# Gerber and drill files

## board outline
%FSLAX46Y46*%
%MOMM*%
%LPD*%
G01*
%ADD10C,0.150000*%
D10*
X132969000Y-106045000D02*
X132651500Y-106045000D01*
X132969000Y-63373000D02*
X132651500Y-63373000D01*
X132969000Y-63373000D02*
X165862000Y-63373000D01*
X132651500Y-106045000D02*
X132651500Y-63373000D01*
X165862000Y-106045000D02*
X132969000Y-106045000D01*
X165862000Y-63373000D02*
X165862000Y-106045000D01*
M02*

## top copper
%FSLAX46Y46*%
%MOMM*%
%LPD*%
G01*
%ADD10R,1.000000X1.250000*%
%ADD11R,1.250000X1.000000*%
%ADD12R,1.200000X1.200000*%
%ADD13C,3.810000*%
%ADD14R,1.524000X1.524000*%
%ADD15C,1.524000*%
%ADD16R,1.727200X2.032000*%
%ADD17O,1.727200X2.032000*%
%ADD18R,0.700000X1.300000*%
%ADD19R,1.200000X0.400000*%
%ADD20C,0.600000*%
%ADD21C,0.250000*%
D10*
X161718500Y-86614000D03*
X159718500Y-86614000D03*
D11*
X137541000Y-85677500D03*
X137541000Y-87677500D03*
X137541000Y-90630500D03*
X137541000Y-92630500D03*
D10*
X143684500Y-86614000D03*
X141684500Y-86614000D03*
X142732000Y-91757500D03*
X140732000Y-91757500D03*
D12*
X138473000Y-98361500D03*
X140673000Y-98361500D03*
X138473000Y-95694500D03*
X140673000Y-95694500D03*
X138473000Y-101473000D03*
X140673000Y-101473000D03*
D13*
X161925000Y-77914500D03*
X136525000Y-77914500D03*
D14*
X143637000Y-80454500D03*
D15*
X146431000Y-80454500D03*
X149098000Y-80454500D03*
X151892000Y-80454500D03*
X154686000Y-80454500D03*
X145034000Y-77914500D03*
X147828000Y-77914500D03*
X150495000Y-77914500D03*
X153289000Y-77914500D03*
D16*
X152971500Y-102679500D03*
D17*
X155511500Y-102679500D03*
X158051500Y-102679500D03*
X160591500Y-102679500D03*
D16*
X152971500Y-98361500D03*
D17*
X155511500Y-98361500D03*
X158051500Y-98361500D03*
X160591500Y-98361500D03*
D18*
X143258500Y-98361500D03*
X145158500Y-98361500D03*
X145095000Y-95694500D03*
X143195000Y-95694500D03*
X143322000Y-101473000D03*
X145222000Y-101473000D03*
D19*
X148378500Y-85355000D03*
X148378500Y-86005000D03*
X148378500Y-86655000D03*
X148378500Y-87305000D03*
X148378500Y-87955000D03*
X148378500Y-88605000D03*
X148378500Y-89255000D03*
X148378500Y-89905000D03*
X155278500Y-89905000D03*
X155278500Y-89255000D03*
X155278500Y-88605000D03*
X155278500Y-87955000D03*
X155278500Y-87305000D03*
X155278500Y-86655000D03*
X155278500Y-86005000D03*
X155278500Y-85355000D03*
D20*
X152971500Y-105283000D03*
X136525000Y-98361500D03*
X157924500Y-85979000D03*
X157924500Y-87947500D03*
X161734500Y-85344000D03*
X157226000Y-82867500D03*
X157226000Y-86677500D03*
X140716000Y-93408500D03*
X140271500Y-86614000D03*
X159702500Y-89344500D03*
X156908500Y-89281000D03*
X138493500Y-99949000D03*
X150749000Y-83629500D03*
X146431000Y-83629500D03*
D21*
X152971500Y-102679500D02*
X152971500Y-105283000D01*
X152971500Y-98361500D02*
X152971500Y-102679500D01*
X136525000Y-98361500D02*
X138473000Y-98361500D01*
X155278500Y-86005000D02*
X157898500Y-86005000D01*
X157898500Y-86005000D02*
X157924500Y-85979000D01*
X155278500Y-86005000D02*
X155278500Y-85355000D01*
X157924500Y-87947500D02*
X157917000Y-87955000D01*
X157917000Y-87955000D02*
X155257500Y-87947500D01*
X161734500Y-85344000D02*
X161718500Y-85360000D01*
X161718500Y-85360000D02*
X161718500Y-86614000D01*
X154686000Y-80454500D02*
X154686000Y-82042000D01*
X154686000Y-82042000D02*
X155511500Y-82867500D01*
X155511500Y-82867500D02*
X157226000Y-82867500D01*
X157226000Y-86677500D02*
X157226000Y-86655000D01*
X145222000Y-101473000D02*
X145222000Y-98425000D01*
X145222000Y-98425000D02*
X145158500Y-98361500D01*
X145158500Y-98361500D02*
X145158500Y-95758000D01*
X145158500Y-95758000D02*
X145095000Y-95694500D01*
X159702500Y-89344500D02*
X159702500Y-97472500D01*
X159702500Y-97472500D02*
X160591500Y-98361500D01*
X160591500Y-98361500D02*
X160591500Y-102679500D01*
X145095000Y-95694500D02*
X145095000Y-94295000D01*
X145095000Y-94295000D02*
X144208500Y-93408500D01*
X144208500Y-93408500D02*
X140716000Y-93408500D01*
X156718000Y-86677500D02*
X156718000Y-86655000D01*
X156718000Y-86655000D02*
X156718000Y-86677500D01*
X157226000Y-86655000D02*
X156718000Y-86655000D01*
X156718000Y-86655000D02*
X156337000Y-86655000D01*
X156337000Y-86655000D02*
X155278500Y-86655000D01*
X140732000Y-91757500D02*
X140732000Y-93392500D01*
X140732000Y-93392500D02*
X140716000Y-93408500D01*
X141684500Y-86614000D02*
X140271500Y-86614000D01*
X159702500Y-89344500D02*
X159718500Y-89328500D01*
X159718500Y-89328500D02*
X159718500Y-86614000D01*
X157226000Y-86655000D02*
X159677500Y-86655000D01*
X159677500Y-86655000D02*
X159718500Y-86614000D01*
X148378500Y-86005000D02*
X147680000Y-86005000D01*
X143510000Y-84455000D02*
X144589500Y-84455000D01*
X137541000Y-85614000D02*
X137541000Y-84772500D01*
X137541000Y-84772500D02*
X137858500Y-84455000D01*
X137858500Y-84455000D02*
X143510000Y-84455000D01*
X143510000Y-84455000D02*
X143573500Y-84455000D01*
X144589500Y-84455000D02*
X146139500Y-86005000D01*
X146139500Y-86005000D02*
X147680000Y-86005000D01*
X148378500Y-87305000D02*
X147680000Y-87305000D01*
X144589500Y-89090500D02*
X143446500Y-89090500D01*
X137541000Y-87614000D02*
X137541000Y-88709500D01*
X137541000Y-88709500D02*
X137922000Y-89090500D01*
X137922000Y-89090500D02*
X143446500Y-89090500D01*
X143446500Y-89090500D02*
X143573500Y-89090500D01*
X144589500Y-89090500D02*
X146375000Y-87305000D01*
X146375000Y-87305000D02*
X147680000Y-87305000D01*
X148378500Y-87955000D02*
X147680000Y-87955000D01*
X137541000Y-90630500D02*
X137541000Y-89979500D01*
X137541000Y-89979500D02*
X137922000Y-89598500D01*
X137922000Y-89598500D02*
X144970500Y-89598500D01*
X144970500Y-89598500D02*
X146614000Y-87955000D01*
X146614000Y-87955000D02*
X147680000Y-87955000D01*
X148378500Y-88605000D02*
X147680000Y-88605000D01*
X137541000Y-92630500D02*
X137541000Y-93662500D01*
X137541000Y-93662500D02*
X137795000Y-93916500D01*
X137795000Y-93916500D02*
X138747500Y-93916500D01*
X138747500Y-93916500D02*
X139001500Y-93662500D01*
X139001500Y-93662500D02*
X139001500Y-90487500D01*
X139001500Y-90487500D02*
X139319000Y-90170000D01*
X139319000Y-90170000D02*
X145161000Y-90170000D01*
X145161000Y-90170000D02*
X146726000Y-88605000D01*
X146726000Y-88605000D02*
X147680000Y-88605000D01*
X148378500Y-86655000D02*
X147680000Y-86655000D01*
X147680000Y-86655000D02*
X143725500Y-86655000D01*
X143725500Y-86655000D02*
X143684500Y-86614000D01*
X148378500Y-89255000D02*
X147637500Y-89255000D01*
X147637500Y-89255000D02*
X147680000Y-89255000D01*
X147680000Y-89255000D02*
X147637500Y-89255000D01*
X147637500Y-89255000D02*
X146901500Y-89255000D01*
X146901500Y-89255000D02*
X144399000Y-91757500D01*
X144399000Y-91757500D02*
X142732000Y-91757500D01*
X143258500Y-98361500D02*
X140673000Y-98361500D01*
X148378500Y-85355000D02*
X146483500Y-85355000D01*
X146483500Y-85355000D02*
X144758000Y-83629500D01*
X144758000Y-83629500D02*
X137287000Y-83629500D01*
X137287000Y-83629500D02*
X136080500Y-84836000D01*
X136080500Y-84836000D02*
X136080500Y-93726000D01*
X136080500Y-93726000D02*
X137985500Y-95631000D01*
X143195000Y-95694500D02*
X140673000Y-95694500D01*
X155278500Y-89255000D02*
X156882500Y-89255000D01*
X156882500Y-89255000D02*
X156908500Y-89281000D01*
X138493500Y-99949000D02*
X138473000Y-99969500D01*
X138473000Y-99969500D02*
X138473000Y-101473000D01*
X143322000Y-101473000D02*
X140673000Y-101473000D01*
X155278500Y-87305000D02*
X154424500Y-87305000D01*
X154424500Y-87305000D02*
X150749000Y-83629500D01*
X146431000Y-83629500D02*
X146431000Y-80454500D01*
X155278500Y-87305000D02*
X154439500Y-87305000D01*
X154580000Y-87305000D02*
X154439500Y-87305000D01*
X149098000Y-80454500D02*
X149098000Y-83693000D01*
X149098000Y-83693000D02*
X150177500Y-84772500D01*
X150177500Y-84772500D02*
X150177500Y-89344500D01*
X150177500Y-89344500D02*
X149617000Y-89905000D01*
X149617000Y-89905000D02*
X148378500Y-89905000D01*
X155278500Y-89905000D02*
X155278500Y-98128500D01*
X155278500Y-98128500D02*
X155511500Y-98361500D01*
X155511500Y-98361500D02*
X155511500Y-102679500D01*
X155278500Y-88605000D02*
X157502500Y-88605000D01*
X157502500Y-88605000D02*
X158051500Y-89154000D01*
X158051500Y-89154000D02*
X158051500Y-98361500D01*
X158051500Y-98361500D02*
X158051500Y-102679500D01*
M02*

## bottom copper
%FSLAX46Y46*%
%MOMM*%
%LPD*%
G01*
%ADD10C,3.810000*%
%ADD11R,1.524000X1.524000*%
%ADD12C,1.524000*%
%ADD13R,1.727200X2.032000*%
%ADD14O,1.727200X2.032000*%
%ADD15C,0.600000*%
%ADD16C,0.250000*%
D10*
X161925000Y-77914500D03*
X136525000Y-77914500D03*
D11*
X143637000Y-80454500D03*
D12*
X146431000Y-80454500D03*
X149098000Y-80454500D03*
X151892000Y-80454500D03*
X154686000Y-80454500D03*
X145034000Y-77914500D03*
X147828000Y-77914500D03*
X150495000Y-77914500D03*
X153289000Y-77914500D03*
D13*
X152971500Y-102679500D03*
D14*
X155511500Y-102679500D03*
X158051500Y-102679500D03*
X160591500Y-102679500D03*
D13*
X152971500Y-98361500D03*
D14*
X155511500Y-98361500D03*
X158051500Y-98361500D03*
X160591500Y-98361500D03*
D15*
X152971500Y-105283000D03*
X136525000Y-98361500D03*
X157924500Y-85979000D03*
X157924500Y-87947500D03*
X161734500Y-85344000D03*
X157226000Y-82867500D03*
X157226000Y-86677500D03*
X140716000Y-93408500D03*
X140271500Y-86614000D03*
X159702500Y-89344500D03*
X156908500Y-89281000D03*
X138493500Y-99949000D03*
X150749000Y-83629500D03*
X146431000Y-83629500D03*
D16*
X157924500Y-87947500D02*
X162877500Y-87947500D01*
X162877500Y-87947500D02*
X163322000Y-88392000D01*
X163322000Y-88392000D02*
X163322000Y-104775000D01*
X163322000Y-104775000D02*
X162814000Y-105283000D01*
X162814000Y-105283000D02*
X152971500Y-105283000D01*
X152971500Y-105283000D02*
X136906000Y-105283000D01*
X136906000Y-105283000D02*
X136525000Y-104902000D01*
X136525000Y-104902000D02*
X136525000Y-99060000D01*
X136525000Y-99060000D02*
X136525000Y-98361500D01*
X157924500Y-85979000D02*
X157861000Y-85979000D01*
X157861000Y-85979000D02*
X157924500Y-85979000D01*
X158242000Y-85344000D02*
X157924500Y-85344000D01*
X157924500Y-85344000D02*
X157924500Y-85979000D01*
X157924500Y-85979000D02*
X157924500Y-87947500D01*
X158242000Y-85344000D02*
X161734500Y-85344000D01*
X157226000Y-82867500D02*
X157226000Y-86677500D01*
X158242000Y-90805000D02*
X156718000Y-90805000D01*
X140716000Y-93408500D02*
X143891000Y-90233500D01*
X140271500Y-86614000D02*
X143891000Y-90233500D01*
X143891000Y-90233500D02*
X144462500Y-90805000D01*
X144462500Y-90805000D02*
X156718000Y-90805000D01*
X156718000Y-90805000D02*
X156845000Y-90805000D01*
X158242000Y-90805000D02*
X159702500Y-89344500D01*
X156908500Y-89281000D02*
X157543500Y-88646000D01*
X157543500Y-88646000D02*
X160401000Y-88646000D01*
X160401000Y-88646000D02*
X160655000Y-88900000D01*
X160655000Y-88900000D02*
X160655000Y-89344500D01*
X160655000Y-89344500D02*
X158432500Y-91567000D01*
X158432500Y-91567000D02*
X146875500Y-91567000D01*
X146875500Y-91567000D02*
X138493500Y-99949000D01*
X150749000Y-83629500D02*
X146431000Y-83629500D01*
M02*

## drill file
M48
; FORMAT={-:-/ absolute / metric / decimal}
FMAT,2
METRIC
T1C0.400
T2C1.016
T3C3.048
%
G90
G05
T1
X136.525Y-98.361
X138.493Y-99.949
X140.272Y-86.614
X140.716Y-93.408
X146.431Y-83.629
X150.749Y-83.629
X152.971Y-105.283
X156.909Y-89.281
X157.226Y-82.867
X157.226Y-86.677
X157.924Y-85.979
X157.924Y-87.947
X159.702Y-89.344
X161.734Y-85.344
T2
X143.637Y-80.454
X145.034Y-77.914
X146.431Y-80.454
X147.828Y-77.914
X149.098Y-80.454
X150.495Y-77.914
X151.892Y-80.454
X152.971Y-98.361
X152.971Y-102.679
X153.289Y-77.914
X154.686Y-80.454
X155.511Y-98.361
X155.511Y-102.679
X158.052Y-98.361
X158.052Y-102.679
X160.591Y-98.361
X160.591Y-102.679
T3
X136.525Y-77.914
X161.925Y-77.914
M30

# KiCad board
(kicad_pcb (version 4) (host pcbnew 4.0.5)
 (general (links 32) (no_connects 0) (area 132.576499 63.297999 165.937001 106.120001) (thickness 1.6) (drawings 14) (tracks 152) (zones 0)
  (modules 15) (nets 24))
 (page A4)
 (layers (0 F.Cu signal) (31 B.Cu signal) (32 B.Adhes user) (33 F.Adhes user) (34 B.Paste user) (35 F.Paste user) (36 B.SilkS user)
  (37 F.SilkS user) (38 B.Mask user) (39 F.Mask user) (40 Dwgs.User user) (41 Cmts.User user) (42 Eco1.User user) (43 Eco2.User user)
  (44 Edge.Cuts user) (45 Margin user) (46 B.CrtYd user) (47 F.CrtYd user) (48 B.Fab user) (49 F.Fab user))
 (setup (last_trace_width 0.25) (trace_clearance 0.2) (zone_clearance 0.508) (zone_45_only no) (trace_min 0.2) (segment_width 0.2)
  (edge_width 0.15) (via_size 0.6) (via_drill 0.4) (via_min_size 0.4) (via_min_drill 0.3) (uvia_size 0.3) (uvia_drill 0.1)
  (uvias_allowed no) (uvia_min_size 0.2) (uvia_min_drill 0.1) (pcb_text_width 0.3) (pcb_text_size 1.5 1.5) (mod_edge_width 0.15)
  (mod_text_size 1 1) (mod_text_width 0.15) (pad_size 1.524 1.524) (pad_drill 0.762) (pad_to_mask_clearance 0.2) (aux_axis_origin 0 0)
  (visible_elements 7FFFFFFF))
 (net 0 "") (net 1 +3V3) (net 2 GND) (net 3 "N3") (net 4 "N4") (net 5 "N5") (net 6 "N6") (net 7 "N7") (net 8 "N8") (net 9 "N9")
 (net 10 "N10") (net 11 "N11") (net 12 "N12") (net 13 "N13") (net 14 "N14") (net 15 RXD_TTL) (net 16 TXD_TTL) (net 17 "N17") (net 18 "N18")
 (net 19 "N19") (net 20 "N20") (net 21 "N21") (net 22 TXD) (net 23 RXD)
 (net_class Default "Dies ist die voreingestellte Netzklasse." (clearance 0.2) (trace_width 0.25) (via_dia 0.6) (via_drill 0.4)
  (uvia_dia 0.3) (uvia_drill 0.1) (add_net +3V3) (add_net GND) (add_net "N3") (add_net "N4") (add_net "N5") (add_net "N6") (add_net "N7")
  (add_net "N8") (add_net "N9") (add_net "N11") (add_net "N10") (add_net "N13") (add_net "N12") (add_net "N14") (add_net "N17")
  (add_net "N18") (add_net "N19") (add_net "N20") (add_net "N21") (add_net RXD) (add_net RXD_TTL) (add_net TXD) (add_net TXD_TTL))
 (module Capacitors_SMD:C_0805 (layer F.Cu) (at 160.7185 86.614 180)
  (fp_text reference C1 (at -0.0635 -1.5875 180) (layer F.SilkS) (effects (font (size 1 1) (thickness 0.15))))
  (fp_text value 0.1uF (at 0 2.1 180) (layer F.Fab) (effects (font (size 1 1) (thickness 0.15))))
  (pad 1 smd rect (at -1 0 180) (size 1 1.25) (layers F.Cu F.Paste F.Mask) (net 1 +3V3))
  (pad 2 smd rect (at 1 0 180) (size 1 1.25) (layers F.Cu F.Paste F.Mask) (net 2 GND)))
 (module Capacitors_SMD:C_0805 (layer F.Cu) (at 137.541 86.6775 270)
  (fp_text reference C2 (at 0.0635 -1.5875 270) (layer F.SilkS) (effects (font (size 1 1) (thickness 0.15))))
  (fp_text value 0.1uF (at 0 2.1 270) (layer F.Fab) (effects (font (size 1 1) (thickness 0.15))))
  (pad 1 smd rect (at -1 0 270) (size 1 1.25) (layers F.Cu F.Paste F.Mask) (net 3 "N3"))
  (pad 2 smd rect (at 1 0 270) (size 1 1.25) (layers F.Cu F.Paste F.Mask) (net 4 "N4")))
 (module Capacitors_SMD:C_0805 (layer F.Cu) (at 137.541 91.6305 270)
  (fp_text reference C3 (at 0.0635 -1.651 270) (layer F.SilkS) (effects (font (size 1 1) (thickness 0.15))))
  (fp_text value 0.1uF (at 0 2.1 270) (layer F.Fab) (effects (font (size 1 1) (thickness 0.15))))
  (pad 1 smd rect (at -1 0 270) (size 1 1.25) (layers F.Cu F.Paste F.Mask) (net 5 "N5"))
  (pad 2 smd rect (at 1 0 270) (size 1 1.25) (layers F.Cu F.Paste F.Mask) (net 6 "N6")))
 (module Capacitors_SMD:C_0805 (layer F.Cu) (at 142.6845 86.614 180)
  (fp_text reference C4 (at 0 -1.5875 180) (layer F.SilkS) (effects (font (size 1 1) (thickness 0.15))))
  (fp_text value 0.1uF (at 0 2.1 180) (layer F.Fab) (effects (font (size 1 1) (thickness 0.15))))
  (pad 1 smd rect (at -1 0 180) (size 1 1.25) (layers F.Cu F.Paste F.Mask) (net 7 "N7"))
  (pad 2 smd rect (at 1 0 180) (size 1 1.25) (layers F.Cu F.Paste F.Mask) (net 2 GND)))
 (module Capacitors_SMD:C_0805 (layer F.Cu) (at 141.732 91.7575 180)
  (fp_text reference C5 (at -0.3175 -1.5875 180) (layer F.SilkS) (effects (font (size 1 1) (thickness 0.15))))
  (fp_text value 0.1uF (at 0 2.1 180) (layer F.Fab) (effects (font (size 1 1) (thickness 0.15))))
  (pad 1 smd rect (at -1 0 180) (size 1 1.25) (layers F.Cu F.Paste F.Mask) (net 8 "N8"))
  (pad 2 smd rect (at 1 0 180) (size 1 1.25) (layers F.Cu F.Paste F.Mask) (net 2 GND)))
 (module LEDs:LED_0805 (layer F.Cu) (at 139.573 98.3615 180)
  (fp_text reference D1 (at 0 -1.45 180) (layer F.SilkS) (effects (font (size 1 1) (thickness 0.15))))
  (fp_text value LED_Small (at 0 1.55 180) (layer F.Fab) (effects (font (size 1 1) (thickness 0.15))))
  (pad 2 smd rect (at 1.1 0) (size 1.2 1.2) (layers F.Cu F.Paste F.Mask) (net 1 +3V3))
  (pad 1 smd rect (at -1.1 0) (size 1.2 1.2) (layers F.Cu F.Paste F.Mask) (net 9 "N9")))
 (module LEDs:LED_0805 (layer F.Cu) (at 139.573 95.6945 180)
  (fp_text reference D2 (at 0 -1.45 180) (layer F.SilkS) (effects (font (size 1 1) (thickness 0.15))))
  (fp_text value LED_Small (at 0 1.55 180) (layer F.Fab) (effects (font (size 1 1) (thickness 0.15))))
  (pad 2 smd rect (at 1.1 0) (size 1.2 1.2) (layers F.Cu F.Paste F.Mask) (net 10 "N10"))
  (pad 1 smd rect (at -1.1 0) (size 1.2 1.2) (layers F.Cu F.Paste F.Mask) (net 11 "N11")))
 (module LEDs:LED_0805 (layer F.Cu) (at 139.573 101.473 180)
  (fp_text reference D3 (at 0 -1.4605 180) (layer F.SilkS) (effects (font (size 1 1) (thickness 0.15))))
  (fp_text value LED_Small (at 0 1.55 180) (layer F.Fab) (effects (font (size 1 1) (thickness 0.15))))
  (pad 2 smd rect (at 1.1 0) (size 1.2 1.2) (layers F.Cu F.Paste F.Mask) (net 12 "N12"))
  (pad 1 smd rect (at -1.1 0) (size 1.2 1.2) (layers F.Cu F.Paste F.Mask) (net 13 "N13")))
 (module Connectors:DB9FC (layer F.Cu) (at 149.098 79.1845)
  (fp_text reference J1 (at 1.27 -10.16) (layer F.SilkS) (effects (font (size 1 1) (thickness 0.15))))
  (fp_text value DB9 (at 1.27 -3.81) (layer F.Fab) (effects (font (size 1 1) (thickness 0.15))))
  (pad "" thru_hole circle (at 12.827 -1.27) (size 3.81 3.81) (drill 3.048) (layers *.Cu *.Mask))
  (pad "" thru_hole circle (at -12.573 -1.27) (size 3.81 3.81) (drill 3.048) (layers *.Cu *.Mask))
  (pad 1 thru_hole rect (at -5.461 1.27) (size 1.524 1.524) (drill 1.016) (layers *.Cu *.Mask) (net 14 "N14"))
  (pad 2 thru_hole circle (at -2.667 1.27) (size 1.524 1.524) (drill 1.016) (layers *.Cu *.Mask) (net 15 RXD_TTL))
  (pad 3 thru_hole circle (at 0 1.27) (size 1.524 1.524) (drill 1.016) (layers *.Cu *.Mask) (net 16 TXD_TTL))
  (pad 4 thru_hole circle (at 2.794 1.27) (size 1.524 1.524) (drill 1.016) (layers *.Cu *.Mask) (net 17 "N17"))
  (pad 5 thru_hole circle (at 5.588 1.27) (size 1.524 1.524) (drill 1.016) (layers *.Cu *.Mask) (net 2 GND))
  (pad 6 thru_hole circle (at -4.064 -1.27) (size 1.524 1.524) (drill 1.016) (layers *.Cu *.Mask) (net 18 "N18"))
  (pad 7 thru_hole circle (at -1.27 -1.27) (size 1.524 1.524) (drill 1.016) (layers *.Cu *.Mask) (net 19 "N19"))
  (pad 8 thru_hole circle (at 1.397 -1.27) (size 1.524 1.524) (drill 1.016) (layers *.Cu *.Mask) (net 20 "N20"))
  (pad 9 thru_hole circle (at 4.191 -1.27) (size 1.524 1.524) (drill 1.016) (layers *.Cu *.Mask) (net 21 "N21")))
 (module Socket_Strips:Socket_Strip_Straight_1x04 (layer F.Cu) (at 152.9715 102.6795)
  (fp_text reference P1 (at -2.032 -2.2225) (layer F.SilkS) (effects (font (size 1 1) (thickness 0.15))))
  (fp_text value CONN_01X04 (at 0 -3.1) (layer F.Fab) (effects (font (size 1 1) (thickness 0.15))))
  (pad 1 thru_hole rect (at 0 0) (size 1.7272 2.032) (drill 1.016) (layers *.Cu *.Mask) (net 1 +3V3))
  (pad 2 thru_hole oval (at 2.54 0) (size 1.7272 2.032) (drill 1.016) (layers *.Cu *.Mask) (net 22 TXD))
  (pad 3 thru_hole oval (at 5.08 0) (size 1.7272 2.032) (drill 1.016) (layers *.Cu *.Mask) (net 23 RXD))
  (pad 4 thru_hole oval (at 7.62 0) (size 1.7272 2.032) (drill 1.016) (layers *.Cu *.Mask) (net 2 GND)))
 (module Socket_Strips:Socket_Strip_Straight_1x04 (layer F.Cu) (at 152.9715 98.3615)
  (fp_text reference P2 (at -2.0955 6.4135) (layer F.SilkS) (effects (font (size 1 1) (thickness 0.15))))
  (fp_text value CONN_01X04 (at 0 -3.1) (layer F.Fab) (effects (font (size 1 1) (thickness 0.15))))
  (pad 1 thru_hole rect (at 0 0) (size 1.7272 2.032) (drill 1.016) (layers *.Cu *.Mask) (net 1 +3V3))
  (pad 2 thru_hole oval (at 2.54 0) (size 1.7272 2.032) (drill 1.016) (layers *.Cu *.Mask) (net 22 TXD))
  (pad 3 thru_hole oval (at 5.08 0) (size 1.7272 2.032) (drill 1.016) (layers *.Cu *.Mask) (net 23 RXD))
  (pad 4 thru_hole oval (at 7.62 0) (size 1.7272 2.032) (drill 1.016) (layers *.Cu *.Mask) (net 2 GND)))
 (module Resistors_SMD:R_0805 (layer F.Cu) (at 144.2085 98.3615)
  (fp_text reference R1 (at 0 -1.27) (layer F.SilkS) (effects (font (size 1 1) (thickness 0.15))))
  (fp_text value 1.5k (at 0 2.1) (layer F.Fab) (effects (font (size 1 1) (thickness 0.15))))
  (pad 1 smd rect (at -0.95 0) (size 0.7 1.3) (layers F.Cu F.Paste F.Mask) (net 9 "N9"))
  (pad 2 smd rect (at 0.95 0) (size 0.7 1.3) (layers F.Cu F.Paste F.Mask) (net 2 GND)))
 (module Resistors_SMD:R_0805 (layer F.Cu) (at 144.145 95.6945 180)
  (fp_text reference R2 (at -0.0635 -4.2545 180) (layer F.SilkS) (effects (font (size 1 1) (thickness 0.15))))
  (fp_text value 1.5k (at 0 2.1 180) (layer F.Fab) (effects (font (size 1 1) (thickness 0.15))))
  (pad 1 smd rect (at -0.95 0 180) (size 0.7 1.3) (layers F.Cu F.Paste F.Mask) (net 2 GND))
  (pad 2 smd rect (at 0.95 0 180) (size 0.7 1.3) (layers F.Cu F.Paste F.Mask) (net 11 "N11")))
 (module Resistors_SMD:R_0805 (layer F.Cu) (at 144.272 101.473)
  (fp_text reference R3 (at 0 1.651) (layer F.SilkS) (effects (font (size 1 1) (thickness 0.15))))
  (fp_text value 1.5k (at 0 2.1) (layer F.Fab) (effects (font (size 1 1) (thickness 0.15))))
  (pad 1 smd rect (at -0.95 0) (size 0.7 1.3) (layers F.Cu F.Paste F.Mask) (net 13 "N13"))
  (pad 2 smd rect (at 0.95 0) (size 0.7 1.3) (layers F.Cu F.Paste F.Mask) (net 2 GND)))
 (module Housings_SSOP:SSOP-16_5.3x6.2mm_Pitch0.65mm (layer F.Cu) (at 151.8285 87.63)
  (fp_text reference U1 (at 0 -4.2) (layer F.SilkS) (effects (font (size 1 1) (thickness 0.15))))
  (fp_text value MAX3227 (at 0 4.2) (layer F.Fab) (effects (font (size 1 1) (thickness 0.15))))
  (pad 1 smd rect (at -3.45 -2.275) (size 1.2 0.4) (layers F.Cu F.Paste F.Mask) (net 10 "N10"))
  (pad 2 smd rect (at -3.45 -1.625) (size 1.2 0.4) (layers F.Cu F.Paste F.Mask) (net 3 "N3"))
  (pad 3 smd rect (at -3.45 -0.975) (size 1.2 0.4) (layers F.Cu F.Paste F.Mask) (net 7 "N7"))
  (pad 4 smd rect (at -3.45 -0.325) (size 1.2 0.4) (layers F.Cu F.Paste F.Mask) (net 4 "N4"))
  (pad 5 smd rect (at -3.45 0.325) (size 1.2 0.4) (layers F.Cu F.Paste F.Mask) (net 5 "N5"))
  (pad 6 smd rect (at -3.45 0.975) (size 1.2 0.4) (layers F.Cu F.Paste F.Mask) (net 6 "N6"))
  (pad 7 smd rect (at -3.45 1.625) (size 1.2 0.4) (layers F.Cu F.Paste F.Mask) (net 8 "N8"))
  (pad 8 smd rect (at -3.45 2.275) (size 1.2 0.4) (layers F.Cu F.Paste F.Mask) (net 16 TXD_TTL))
  (pad 9 smd rect (at 3.45 2.275) (size 1.2 0.4) (layers F.Cu F.Paste F.Mask) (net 22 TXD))
  (pad 10 smd rect (at 3.45 1.625) (size 1.2 0.4) (layers F.Cu F.Paste F.Mask) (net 12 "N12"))
  (pad 11 smd rect (at 3.45 0.975) (size 1.2 0.4) (layers F.Cu F.Paste F.Mask) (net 23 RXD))
  (pad 12 smd rect (at 3.45 0.325) (size 1.2 0.4) (layers F.Cu F.Paste F.Mask) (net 1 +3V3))
  (pad 13 smd rect (at 3.45 -0.325) (size 1.2 0.4) (layers F.Cu F.Paste F.Mask) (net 15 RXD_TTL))
  (pad 14 smd rect (at 3.45 -0.975) (size 1.2 0.4) (layers F.Cu F.Paste F.Mask) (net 2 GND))
  (pad 15 smd rect (at 3.45 -1.625) (size 1.2 0.4) (layers F.Cu F.Paste F.Mask) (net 1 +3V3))
  (pad 16 smd rect (at 3.45 -2.275) (size 1.2 0.4) (layers F.Cu F.Paste F.Mask) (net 1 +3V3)))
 (gr_line (start 132.969 106.045) (end 132.6515 106.045) (angle 90) (layer Edge.Cuts) (width 0.15))
 (gr_line (start 132.969 63.373) (end 132.6515 63.373) (angle 90) (layer Edge.Cuts) (width 0.15))
 (gr_line (start 132.969 63.373) (end 165.862 63.373) (angle 90) (layer Edge.Cuts) (width 0.15))
 (gr_line (start 132.6515 106.045) (end 132.6515 63.373) (angle 90) (layer Edge.Cuts) (width 0.15))
 (gr_line (start 165.862 106.045) (end 132.969 106.045) (angle 90) (layer Edge.Cuts) (width 0.15))
 (gr_line (start 165.862 63.373) (end 165.862 106.045) (angle 90) (layer Edge.Cuts) (width 0.15))
 (segment (start 152.9715 102.6795) (end 152.9715 105.283) (width 0.25) (layer F.Cu) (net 1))
 (via (at 152.9715 105.283) (size 0.6) (drill 0.4) (layers F.Cu B.Cu) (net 1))
 (segment (start 152.9715 98.3615) (end 152.9715 102.6795) (width 0.25) (layer F.Cu) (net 1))
 (segment (start 157.9245 87.9475) (end 162.8775 87.9475) (width 0.25) (layer B.Cu) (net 1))
 (segment (start 162.8775 87.9475) (end 163.322 88.392) (width 0.25) (layer B.Cu) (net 1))
 (segment (start 163.322 88.392) (end 163.322 104.775) (width 0.25) (layer B.Cu) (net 1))
 (segment (start 163.322 104.775) (end 162.814 105.283) (width 0.25) (layer B.Cu) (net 1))
 (segment (start 162.814 105.283) (end 152.9715 105.283) (width 0.25) (layer B.Cu) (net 1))
 (segment (start 152.9715 105.283) (end 136.906 105.283) (width 0.25) (layer B.Cu) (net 1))
 (segment (start 136.906 105.283) (end 136.525 104.902) (width 0.25) (layer B.Cu) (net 1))
 (segment (start 136.525 104.902) (end 136.525 99.06) (width 0.25) (layer B.Cu) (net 1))
 (segment (start 136.525 99.06) (end 136.525 98.3615) (width 0.25) (layer B.Cu) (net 1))
 (via (at 136.525 98.3615) (size 0.6) (drill 0.4) (layers F.Cu B.Cu) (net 1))
 (segment (start 136.525 98.3615) (end 138.473 98.3615) (width 0.25) (layer F.Cu) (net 1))
 (segment (start 155.2785 86.005) (end 157.8985 86.005) (width 0.25) (layer F.Cu) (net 1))
 (segment (start 157.8985 86.005) (end 157.9245 85.979) (width 0.25) (layer F.Cu) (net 1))
 (via (at 157.9245 85.979) (size 0.6) (drill 0.4) (layers F.Cu B.Cu) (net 1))
 (segment (start 157.9245 85.979) (end 157.861 85.979) (width 0.25) (layer B.Cu) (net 1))
 (segment (start 157.861 85.979) (end 157.9245 85.979) (width 0.25) (layer B.Cu) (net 1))
 (segment (start 155.2785 86.005) (end 155.2785 85.355) (width 0.25) (layer F.Cu) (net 1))
 (segment (start 158.242 85.344) (end 157.9245 85.344) (width 0.25) (layer B.Cu) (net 1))
 (segment (start 157.9245 85.344) (end 157.9245 85.979) (width 0.25) (layer B.Cu) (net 1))
 (segment (start 157.9245 85.979) (end 157.9245 87.9475) (width 0.25) (layer B.Cu) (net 1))
 (via (at 157.9245 87.9475) (size 0.6) (drill 0.4) (layers F.Cu B.Cu) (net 1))
 (segment (start 157.9245 87.9475) (end 157.917 87.955) (width 0.25) (layer F.Cu) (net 1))
 (segment (start 157.917 87.955) (end 155.2575 87.9475) (width 0.25) (layer F.Cu) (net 1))
 (segment (start 158.242 85.344) (end 161.7345 85.344) (width 0.25) (layer B.Cu) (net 1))
 (via (at 161.7345 85.344) (size 0.6) (drill 0.4) (layers F.Cu B.Cu) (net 1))
 (segment (start 161.7345 85.344) (end 161.7185 85.36) (width 0.25) (layer F.Cu) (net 1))
 (segment (start 161.7185 85.36) (end 161.7185 86.614) (width 0.25) (layer F.Cu) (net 1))
 (segment (start 154.686 80.4545) (end 154.686 82.042) (width 0.25) (layer F.Cu) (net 2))
 (segment (start 154.686 82.042) (end 155.5115 82.8675) (width 0.25) (layer F.Cu) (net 2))
 (segment (start 155.5115 82.8675) (end 157.226 82.8675) (width 0.25) (layer F.Cu) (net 2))
 (via (at 157.226 82.8675) (size 0.6) (drill 0.4) (layers F.Cu B.Cu) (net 2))
 (segment (start 157.226 82.8675) (end 157.226 86.6775) (width 0.25) (layer B.Cu) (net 2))
 (via (at 157.226 86.6775) (size 0.6) (drill 0.4) (layers F.Cu B.Cu) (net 2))
 (segment (start 157.226 86.6775) (end 157.226 86.655) (width 0.25) (layer F.Cu) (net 2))
 (segment (start 145.222 101.473) (end 145.222 98.425) (width 0.25) (layer F.Cu) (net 2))
 (segment (start 145.222 98.425) (end 145.1585 98.3615) (width 0.25) (layer F.Cu) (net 2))
 (segment (start 145.1585 98.3615) (end 145.1585 95.758) (width 0.25) (layer F.Cu) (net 2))
 (segment (start 145.1585 95.758) (end 145.095 95.6945) (width 0.25) (layer F.Cu) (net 2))
 (segment (start 159.7025 89.3445) (end 159.7025 97.4725) (width 0.25) (layer F.Cu) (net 2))
 (segment (start 159.7025 97.4725) (end 160.5915 98.3615) (width 0.25) (layer F.Cu) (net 2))
 (segment (start 160.5915 98.3615) (end 160.5915 102.6795) (width 0.25) (layer F.Cu) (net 2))
 (segment (start 145.095 95.6945) (end 145.095 94.295) (width 0.25) (layer F.Cu) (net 2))
 (segment (start 145.095 94.295) (end 144.2085 93.4085) (width 0.25) (layer F.Cu) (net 2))
 (segment (start 144.2085 93.4085) (end 140.716 93.4085) (width 0.25) (layer F.Cu) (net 2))
 (segment (start 156.718 86.6775) (end 156.718 86.655) (width 0.25) (layer F.Cu) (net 2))
 (segment (start 156.718 86.655) (end 156.718 86.6775) (width 0.25) (layer F.Cu) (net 2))
 (segment (start 157.226 86.655) (end 156.718 86.655) (width 0.25) (layer F.Cu) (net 2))
 (segment (start 156.718 86.655) (end 156.337 86.655) (width 0.25) (layer F.Cu) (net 2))
 (segment (start 156.337 86.655) (end 155.2785 86.655) (width 0.25) (layer F.Cu) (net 2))
 (segment (start 158.242 90.805) (end 156.718 90.805) (width 0.25) (layer B.Cu) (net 2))
 (segment (start 140.732 91.7575) (end 140.732 93.3925) (width 0.25) (layer F.Cu) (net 2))
 (segment (start 140.732 93.3925) (end 140.716 93.4085) (width 0.25) (layer F.Cu) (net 2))
 (via (at 140.716 93.4085) (size 0.6) (drill 0.4) (layers F.Cu B.Cu) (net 2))
 (segment (start 140.716 93.4085) (end 143.891 90.2335) (width 0.25) (layer B.Cu) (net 2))
 (segment (start 141.6845 86.614) (end 140.2715 86.614) (width 0.25) (layer F.Cu) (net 2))
 (via (at 140.2715 86.614) (size 0.6) (drill 0.4) (layers F.Cu B.Cu) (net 2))
 (segment (start 140.2715 86.614) (end 143.891 90.2335) (width 0.25) (layer B.Cu) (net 2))
 (segment (start 143.891 90.2335) (end 144.4625 90.805) (width 0.25) (layer B.Cu) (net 2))
 (segment (start 144.4625 90.805) (end 156.718 90.805) (width 0.25) (layer B.Cu) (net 2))
 (segment (start 156.718 90.805) (end 156.845 90.805) (width 0.25) (layer B.Cu) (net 2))
 (segment (start 158.242 90.805) (end 159.7025 89.3445) (width 0.25) (layer B.Cu) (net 2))
 (via (at 159.7025 89.3445) (size 0.6) (drill 0.4) (layers F.Cu B.Cu) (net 2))
 (segment (start 159.7025 89.3445) (end 159.7185 89.3285) (width 0.25) (layer F.Cu) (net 2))
 (segment (start 159.7185 89.3285) (end 159.7185 86.614) (width 0.25) (layer F.Cu) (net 2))
 (segment (start 157.226 86.655) (end 159.6775 86.655) (width 0.25) (layer F.Cu) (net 2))
 (segment (start 159.6775 86.655) (end 159.7185 86.614) (width 0.25) (layer F.Cu) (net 2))
 (segment (start 148.3785 86.005) (end 147.68 86.005) (width 0.25) (layer F.Cu) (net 3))
 (segment (start 143.51 84.455) (end 144.5895 84.455) (width 0.25) (layer F.Cu) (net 3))
 (segment (start 137.541 85.614) (end 137.541 84.7725) (width 0.25) (layer F.Cu) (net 3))
 (segment (start 137.541 84.7725) (end 137.8585 84.455) (width 0.25) (layer F.Cu) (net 3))
 (segment (start 137.8585 84.455) (end 143.51 84.455) (width 0.25) (layer F.Cu) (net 3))
 (segment (start 143.51 84.455) (end 143.5735 84.455) (width 0.25) (layer F.Cu) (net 3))
 (segment (start 144.5895 84.455) (end 146.1395 86.005) (width 0.25) (layer F.Cu) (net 3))
 (segment (start 146.1395 86.005) (end 147.68 86.005) (width 0.25) (layer F.Cu) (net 3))
 (segment (start 148.3785 87.305) (end 147.68 87.305) (width 0.25) (layer F.Cu) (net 4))
 (segment (start 144.5895 89.0905) (end 143.4465 89.0905) (width 0.25) (layer F.Cu) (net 4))
 (segment (start 137.541 87.614) (end 137.541 88.7095) (width 0.25) (layer F.Cu) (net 4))
 (segment (start 137.541 88.7095) (end 137.922 89.0905) (width 0.25) (layer F.Cu) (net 4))
 (segment (start 137.922 89.0905) (end 143.4465 89.0905) (width 0.25) (layer F.Cu) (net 4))
 (segment (start 143.4465 89.0905) (end 143.5735 89.0905) (width 0.25) (layer F.Cu) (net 4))
 (segment (start 144.5895 89.0905) (end 146.375 87.305) (width 0.25) (layer F.Cu) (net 4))
 (segment (start 146.375 87.305) (end 147.68 87.305) (width 0.25) (layer F.Cu) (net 4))
 (segment (start 148.3785 87.955) (end 147.68 87.955) (width 0.25) (layer F.Cu) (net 5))
 (segment (start 137.541 90.6305) (end 137.541 89.9795) (width 0.25) (layer F.Cu) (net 5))
 (segment (start 137.541 89.9795) (end 137.922 89.5985) (width 0.25) (layer F.Cu) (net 5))
 (segment (start 137.922 89.5985) (end 144.9705 89.5985) (width 0.25) (layer F.Cu) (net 5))
 (segment (start 144.9705 89.5985) (end 146.614 87.955) (width 0.25) (layer F.Cu) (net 5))
 (segment (start 146.614 87.955) (end 147.68 87.955) (width 0.25) (layer F.Cu) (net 5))
 (segment (start 148.3785 88.605) (end 147.68 88.605) (width 0.25) (layer F.Cu) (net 6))
 (segment (start 137.541 92.6305) (end 137.541 93.6625) (width 0.25) (layer F.Cu) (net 6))
 (segment (start 137.541 93.6625) (end 137.795 93.9165) (width 0.25) (layer F.Cu) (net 6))
 (segment (start 137.795 93.9165) (end 138.7475 93.9165) (width 0.25) (layer F.Cu) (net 6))
 (segment (start 138.7475 93.9165) (end 139.0015 93.6625) (width 0.25) (layer F.Cu) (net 6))
 (segment (start 139.0015 93.6625) (end 139.0015 90.4875) (width 0.25) (layer F.Cu) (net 6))
 (segment (start 139.0015 90.4875) (end 139.319 90.17) (width 0.25) (layer F.Cu) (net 6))
 (segment (start 139.319 90.17) (end 145.161 90.17) (width 0.25) (layer F.Cu) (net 6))
 (segment (start 145.161 90.17) (end 146.726 88.605) (width 0.25) (layer F.Cu) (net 6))
 (segment (start 146.726 88.605) (end 147.68 88.605) (width 0.25) (layer F.Cu) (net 6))
 (segment (start 148.3785 86.655) (end 147.68 86.655) (width 0.25) (layer F.Cu) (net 7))
 (segment (start 147.68 86.655) (end 143.7255 86.655) (width 0.25) (layer F.Cu) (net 7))
 (segment (start 143.7255 86.655) (end 143.6845 86.614) (width 0.25) (layer F.Cu) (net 7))
 (segment (start 148.3785 89.255) (end 147.6375 89.255) (width 0.25) (layer F.Cu) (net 8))
 (segment (start 147.6375 89.255) (end 147.68 89.255) (width 0.25) (layer F.Cu) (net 8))
 (segment (start 147.68 89.255) (end 147.6375 89.255) (width 0.25) (layer F.Cu) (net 8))
 (segment (start 147.6375 89.255) (end 146.9015 89.255) (width 0.25) (layer F.Cu) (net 8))
 (segment (start 146.9015 89.255) (end 144.399 91.7575) (width 0.25) (layer F.Cu) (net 8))
 (segment (start 144.399 91.7575) (end 142.732 91.7575) (width 0.25) (layer F.Cu) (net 8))
 (segment (start 143.2585 98.3615) (end 140.673 98.3615) (width 0.25) (layer F.Cu) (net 9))
 (segment (start 148.3785 85.355) (end 146.4835 85.355) (width 0.25) (layer F.Cu) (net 10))
 (segment (start 146.4835 85.355) (end 144.758 83.6295) (width 0.25) (layer F.Cu) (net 10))
 (segment (start 144.758 83.6295) (end 137.287 83.6295) (width 0.25) (layer F.Cu) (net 10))
 (segment (start 137.287 83.6295) (end 136.0805 84.836) (width 0.25) (layer F.Cu) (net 10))
 (segment (start 136.0805 84.836) (end 136.0805 93.726) (width 0.25) (layer F.Cu) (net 10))
 (segment (start 136.0805 93.726) (end 137.9855 95.631) (width 0.25) (layer F.Cu) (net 10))
 (segment (start 143.195 95.6945) (end 140.673 95.6945) (width 0.25) (layer F.Cu) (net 11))
 (segment (start 155.2785 89.255) (end 156.8825 89.255) (width 0.25) (layer F.Cu) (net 12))
 (segment (start 156.8825 89.255) (end 156.9085 89.281) (width 0.25) (layer F.Cu) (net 12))
 (via (at 156.9085 89.281) (size 0.6) (drill 0.4) (layers F.Cu B.Cu) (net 12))
 (segment (start 156.9085 89.281) (end 157.5435 88.646) (width 0.25) (layer B.Cu) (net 12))
 (segment (start 157.5435 88.646) (end 160.401 88.646) (width 0.25) (layer B.Cu) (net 12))
 (segment (start 160.401 88.646) (end 160.655 88.9) (width 0.25) (layer B.Cu) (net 12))
 (segment (start 160.655 88.9) (end 160.655 89.3445) (width 0.25) (layer B.Cu) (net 12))
 (segment (start 160.655 89.3445) (end 158.4325 91.567) (width 0.25) (layer B.Cu) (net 12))
 (segment (start 158.4325 91.567) (end 146.8755 91.567) (width 0.25) (layer B.Cu) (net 12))
 (segment (start 146.8755 91.567) (end 138.4935 99.949) (width 0.25) (layer B.Cu) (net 12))
 (via (at 138.4935 99.949) (size 0.6) (drill 0.4) (layers F.Cu B.Cu) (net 12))
 (segment (start 138.4935 99.949) (end 138.473 99.9695) (width 0.25) (layer F.Cu) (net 12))
 (segment (start 138.473 99.9695) (end 138.473 101.473) (width 0.25) (layer F.Cu) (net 12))
 (segment (start 143.322 101.473) (end 140.673 101.473) (width 0.25) (layer F.Cu) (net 13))
 (segment (start 155.2785 87.305) (end 154.4245 87.305) (width 0.25) (layer F.Cu) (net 15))
 (segment (start 154.4245 87.305) (end 150.749 83.6295) (width 0.25) (layer F.Cu) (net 15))
 (via (at 150.749 83.6295) (size 0.6) (drill 0.4) (layers F.Cu B.Cu) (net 15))
 (segment (start 150.749 83.6295) (end 146.431 83.6295) (width 0.25) (layer B.Cu) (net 15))
 (via (at 146.431 83.6295) (size 0.6) (drill 0.4) (layers F.Cu B.Cu) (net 15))
 (segment (start 146.431 83.6295) (end 146.431 80.4545) (width 0.25) (layer F.Cu) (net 15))
 (segment (start 155.2785 87.305) (end 154.4395 87.305) (width 0.25) (layer F.Cu) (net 15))
 (segment (start 154.58 87.305) (end 154.4395 87.305) (width 0.25) (layer F.Cu) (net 15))
 (segment (start 149.098 80.4545) (end 149.098 83.693) (width 0.25) (layer F.Cu) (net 16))
 (segment (start 149.098 83.693) (end 150.1775 84.7725) (width 0.25) (layer F.Cu) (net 16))
 (segment (start 150.1775 84.7725) (end 150.1775 89.3445) (width 0.25) (layer F.Cu) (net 16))
 (segment (start 150.1775 89.3445) (end 149.617 89.905) (width 0.25) (layer F.Cu) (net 16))
 (segment (start 149.617 89.905) (end 148.3785 89.905) (width 0.25) (layer F.Cu) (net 16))
 (segment (start 155.2785 89.905) (end 155.2785 98.1285) (width 0.25) (layer F.Cu) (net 22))
 (segment (start 155.2785 98.1285) (end 155.5115 98.3615) (width 0.25) (layer F.Cu) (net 22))
 (segment (start 155.5115 98.3615) (end 155.5115 102.6795) (width 0.25) (layer F.Cu) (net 22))
 (segment (start 155.2785 88.605) (end 157.5025 88.605) (width 0.25) (layer F.Cu) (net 23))
 (segment (start 157.5025 88.605) (end 158.0515 89.154) (width 0.25) (layer F.Cu) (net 23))
 (segment (start 158.0515 89.154) (end 158.0515 98.3615) (width 0.25) (layer F.Cu) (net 23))
 (segment (start 158.0515 98.3615) (end 158.0515 102.6795) (width 0.25) (layer F.Cu) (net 23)))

